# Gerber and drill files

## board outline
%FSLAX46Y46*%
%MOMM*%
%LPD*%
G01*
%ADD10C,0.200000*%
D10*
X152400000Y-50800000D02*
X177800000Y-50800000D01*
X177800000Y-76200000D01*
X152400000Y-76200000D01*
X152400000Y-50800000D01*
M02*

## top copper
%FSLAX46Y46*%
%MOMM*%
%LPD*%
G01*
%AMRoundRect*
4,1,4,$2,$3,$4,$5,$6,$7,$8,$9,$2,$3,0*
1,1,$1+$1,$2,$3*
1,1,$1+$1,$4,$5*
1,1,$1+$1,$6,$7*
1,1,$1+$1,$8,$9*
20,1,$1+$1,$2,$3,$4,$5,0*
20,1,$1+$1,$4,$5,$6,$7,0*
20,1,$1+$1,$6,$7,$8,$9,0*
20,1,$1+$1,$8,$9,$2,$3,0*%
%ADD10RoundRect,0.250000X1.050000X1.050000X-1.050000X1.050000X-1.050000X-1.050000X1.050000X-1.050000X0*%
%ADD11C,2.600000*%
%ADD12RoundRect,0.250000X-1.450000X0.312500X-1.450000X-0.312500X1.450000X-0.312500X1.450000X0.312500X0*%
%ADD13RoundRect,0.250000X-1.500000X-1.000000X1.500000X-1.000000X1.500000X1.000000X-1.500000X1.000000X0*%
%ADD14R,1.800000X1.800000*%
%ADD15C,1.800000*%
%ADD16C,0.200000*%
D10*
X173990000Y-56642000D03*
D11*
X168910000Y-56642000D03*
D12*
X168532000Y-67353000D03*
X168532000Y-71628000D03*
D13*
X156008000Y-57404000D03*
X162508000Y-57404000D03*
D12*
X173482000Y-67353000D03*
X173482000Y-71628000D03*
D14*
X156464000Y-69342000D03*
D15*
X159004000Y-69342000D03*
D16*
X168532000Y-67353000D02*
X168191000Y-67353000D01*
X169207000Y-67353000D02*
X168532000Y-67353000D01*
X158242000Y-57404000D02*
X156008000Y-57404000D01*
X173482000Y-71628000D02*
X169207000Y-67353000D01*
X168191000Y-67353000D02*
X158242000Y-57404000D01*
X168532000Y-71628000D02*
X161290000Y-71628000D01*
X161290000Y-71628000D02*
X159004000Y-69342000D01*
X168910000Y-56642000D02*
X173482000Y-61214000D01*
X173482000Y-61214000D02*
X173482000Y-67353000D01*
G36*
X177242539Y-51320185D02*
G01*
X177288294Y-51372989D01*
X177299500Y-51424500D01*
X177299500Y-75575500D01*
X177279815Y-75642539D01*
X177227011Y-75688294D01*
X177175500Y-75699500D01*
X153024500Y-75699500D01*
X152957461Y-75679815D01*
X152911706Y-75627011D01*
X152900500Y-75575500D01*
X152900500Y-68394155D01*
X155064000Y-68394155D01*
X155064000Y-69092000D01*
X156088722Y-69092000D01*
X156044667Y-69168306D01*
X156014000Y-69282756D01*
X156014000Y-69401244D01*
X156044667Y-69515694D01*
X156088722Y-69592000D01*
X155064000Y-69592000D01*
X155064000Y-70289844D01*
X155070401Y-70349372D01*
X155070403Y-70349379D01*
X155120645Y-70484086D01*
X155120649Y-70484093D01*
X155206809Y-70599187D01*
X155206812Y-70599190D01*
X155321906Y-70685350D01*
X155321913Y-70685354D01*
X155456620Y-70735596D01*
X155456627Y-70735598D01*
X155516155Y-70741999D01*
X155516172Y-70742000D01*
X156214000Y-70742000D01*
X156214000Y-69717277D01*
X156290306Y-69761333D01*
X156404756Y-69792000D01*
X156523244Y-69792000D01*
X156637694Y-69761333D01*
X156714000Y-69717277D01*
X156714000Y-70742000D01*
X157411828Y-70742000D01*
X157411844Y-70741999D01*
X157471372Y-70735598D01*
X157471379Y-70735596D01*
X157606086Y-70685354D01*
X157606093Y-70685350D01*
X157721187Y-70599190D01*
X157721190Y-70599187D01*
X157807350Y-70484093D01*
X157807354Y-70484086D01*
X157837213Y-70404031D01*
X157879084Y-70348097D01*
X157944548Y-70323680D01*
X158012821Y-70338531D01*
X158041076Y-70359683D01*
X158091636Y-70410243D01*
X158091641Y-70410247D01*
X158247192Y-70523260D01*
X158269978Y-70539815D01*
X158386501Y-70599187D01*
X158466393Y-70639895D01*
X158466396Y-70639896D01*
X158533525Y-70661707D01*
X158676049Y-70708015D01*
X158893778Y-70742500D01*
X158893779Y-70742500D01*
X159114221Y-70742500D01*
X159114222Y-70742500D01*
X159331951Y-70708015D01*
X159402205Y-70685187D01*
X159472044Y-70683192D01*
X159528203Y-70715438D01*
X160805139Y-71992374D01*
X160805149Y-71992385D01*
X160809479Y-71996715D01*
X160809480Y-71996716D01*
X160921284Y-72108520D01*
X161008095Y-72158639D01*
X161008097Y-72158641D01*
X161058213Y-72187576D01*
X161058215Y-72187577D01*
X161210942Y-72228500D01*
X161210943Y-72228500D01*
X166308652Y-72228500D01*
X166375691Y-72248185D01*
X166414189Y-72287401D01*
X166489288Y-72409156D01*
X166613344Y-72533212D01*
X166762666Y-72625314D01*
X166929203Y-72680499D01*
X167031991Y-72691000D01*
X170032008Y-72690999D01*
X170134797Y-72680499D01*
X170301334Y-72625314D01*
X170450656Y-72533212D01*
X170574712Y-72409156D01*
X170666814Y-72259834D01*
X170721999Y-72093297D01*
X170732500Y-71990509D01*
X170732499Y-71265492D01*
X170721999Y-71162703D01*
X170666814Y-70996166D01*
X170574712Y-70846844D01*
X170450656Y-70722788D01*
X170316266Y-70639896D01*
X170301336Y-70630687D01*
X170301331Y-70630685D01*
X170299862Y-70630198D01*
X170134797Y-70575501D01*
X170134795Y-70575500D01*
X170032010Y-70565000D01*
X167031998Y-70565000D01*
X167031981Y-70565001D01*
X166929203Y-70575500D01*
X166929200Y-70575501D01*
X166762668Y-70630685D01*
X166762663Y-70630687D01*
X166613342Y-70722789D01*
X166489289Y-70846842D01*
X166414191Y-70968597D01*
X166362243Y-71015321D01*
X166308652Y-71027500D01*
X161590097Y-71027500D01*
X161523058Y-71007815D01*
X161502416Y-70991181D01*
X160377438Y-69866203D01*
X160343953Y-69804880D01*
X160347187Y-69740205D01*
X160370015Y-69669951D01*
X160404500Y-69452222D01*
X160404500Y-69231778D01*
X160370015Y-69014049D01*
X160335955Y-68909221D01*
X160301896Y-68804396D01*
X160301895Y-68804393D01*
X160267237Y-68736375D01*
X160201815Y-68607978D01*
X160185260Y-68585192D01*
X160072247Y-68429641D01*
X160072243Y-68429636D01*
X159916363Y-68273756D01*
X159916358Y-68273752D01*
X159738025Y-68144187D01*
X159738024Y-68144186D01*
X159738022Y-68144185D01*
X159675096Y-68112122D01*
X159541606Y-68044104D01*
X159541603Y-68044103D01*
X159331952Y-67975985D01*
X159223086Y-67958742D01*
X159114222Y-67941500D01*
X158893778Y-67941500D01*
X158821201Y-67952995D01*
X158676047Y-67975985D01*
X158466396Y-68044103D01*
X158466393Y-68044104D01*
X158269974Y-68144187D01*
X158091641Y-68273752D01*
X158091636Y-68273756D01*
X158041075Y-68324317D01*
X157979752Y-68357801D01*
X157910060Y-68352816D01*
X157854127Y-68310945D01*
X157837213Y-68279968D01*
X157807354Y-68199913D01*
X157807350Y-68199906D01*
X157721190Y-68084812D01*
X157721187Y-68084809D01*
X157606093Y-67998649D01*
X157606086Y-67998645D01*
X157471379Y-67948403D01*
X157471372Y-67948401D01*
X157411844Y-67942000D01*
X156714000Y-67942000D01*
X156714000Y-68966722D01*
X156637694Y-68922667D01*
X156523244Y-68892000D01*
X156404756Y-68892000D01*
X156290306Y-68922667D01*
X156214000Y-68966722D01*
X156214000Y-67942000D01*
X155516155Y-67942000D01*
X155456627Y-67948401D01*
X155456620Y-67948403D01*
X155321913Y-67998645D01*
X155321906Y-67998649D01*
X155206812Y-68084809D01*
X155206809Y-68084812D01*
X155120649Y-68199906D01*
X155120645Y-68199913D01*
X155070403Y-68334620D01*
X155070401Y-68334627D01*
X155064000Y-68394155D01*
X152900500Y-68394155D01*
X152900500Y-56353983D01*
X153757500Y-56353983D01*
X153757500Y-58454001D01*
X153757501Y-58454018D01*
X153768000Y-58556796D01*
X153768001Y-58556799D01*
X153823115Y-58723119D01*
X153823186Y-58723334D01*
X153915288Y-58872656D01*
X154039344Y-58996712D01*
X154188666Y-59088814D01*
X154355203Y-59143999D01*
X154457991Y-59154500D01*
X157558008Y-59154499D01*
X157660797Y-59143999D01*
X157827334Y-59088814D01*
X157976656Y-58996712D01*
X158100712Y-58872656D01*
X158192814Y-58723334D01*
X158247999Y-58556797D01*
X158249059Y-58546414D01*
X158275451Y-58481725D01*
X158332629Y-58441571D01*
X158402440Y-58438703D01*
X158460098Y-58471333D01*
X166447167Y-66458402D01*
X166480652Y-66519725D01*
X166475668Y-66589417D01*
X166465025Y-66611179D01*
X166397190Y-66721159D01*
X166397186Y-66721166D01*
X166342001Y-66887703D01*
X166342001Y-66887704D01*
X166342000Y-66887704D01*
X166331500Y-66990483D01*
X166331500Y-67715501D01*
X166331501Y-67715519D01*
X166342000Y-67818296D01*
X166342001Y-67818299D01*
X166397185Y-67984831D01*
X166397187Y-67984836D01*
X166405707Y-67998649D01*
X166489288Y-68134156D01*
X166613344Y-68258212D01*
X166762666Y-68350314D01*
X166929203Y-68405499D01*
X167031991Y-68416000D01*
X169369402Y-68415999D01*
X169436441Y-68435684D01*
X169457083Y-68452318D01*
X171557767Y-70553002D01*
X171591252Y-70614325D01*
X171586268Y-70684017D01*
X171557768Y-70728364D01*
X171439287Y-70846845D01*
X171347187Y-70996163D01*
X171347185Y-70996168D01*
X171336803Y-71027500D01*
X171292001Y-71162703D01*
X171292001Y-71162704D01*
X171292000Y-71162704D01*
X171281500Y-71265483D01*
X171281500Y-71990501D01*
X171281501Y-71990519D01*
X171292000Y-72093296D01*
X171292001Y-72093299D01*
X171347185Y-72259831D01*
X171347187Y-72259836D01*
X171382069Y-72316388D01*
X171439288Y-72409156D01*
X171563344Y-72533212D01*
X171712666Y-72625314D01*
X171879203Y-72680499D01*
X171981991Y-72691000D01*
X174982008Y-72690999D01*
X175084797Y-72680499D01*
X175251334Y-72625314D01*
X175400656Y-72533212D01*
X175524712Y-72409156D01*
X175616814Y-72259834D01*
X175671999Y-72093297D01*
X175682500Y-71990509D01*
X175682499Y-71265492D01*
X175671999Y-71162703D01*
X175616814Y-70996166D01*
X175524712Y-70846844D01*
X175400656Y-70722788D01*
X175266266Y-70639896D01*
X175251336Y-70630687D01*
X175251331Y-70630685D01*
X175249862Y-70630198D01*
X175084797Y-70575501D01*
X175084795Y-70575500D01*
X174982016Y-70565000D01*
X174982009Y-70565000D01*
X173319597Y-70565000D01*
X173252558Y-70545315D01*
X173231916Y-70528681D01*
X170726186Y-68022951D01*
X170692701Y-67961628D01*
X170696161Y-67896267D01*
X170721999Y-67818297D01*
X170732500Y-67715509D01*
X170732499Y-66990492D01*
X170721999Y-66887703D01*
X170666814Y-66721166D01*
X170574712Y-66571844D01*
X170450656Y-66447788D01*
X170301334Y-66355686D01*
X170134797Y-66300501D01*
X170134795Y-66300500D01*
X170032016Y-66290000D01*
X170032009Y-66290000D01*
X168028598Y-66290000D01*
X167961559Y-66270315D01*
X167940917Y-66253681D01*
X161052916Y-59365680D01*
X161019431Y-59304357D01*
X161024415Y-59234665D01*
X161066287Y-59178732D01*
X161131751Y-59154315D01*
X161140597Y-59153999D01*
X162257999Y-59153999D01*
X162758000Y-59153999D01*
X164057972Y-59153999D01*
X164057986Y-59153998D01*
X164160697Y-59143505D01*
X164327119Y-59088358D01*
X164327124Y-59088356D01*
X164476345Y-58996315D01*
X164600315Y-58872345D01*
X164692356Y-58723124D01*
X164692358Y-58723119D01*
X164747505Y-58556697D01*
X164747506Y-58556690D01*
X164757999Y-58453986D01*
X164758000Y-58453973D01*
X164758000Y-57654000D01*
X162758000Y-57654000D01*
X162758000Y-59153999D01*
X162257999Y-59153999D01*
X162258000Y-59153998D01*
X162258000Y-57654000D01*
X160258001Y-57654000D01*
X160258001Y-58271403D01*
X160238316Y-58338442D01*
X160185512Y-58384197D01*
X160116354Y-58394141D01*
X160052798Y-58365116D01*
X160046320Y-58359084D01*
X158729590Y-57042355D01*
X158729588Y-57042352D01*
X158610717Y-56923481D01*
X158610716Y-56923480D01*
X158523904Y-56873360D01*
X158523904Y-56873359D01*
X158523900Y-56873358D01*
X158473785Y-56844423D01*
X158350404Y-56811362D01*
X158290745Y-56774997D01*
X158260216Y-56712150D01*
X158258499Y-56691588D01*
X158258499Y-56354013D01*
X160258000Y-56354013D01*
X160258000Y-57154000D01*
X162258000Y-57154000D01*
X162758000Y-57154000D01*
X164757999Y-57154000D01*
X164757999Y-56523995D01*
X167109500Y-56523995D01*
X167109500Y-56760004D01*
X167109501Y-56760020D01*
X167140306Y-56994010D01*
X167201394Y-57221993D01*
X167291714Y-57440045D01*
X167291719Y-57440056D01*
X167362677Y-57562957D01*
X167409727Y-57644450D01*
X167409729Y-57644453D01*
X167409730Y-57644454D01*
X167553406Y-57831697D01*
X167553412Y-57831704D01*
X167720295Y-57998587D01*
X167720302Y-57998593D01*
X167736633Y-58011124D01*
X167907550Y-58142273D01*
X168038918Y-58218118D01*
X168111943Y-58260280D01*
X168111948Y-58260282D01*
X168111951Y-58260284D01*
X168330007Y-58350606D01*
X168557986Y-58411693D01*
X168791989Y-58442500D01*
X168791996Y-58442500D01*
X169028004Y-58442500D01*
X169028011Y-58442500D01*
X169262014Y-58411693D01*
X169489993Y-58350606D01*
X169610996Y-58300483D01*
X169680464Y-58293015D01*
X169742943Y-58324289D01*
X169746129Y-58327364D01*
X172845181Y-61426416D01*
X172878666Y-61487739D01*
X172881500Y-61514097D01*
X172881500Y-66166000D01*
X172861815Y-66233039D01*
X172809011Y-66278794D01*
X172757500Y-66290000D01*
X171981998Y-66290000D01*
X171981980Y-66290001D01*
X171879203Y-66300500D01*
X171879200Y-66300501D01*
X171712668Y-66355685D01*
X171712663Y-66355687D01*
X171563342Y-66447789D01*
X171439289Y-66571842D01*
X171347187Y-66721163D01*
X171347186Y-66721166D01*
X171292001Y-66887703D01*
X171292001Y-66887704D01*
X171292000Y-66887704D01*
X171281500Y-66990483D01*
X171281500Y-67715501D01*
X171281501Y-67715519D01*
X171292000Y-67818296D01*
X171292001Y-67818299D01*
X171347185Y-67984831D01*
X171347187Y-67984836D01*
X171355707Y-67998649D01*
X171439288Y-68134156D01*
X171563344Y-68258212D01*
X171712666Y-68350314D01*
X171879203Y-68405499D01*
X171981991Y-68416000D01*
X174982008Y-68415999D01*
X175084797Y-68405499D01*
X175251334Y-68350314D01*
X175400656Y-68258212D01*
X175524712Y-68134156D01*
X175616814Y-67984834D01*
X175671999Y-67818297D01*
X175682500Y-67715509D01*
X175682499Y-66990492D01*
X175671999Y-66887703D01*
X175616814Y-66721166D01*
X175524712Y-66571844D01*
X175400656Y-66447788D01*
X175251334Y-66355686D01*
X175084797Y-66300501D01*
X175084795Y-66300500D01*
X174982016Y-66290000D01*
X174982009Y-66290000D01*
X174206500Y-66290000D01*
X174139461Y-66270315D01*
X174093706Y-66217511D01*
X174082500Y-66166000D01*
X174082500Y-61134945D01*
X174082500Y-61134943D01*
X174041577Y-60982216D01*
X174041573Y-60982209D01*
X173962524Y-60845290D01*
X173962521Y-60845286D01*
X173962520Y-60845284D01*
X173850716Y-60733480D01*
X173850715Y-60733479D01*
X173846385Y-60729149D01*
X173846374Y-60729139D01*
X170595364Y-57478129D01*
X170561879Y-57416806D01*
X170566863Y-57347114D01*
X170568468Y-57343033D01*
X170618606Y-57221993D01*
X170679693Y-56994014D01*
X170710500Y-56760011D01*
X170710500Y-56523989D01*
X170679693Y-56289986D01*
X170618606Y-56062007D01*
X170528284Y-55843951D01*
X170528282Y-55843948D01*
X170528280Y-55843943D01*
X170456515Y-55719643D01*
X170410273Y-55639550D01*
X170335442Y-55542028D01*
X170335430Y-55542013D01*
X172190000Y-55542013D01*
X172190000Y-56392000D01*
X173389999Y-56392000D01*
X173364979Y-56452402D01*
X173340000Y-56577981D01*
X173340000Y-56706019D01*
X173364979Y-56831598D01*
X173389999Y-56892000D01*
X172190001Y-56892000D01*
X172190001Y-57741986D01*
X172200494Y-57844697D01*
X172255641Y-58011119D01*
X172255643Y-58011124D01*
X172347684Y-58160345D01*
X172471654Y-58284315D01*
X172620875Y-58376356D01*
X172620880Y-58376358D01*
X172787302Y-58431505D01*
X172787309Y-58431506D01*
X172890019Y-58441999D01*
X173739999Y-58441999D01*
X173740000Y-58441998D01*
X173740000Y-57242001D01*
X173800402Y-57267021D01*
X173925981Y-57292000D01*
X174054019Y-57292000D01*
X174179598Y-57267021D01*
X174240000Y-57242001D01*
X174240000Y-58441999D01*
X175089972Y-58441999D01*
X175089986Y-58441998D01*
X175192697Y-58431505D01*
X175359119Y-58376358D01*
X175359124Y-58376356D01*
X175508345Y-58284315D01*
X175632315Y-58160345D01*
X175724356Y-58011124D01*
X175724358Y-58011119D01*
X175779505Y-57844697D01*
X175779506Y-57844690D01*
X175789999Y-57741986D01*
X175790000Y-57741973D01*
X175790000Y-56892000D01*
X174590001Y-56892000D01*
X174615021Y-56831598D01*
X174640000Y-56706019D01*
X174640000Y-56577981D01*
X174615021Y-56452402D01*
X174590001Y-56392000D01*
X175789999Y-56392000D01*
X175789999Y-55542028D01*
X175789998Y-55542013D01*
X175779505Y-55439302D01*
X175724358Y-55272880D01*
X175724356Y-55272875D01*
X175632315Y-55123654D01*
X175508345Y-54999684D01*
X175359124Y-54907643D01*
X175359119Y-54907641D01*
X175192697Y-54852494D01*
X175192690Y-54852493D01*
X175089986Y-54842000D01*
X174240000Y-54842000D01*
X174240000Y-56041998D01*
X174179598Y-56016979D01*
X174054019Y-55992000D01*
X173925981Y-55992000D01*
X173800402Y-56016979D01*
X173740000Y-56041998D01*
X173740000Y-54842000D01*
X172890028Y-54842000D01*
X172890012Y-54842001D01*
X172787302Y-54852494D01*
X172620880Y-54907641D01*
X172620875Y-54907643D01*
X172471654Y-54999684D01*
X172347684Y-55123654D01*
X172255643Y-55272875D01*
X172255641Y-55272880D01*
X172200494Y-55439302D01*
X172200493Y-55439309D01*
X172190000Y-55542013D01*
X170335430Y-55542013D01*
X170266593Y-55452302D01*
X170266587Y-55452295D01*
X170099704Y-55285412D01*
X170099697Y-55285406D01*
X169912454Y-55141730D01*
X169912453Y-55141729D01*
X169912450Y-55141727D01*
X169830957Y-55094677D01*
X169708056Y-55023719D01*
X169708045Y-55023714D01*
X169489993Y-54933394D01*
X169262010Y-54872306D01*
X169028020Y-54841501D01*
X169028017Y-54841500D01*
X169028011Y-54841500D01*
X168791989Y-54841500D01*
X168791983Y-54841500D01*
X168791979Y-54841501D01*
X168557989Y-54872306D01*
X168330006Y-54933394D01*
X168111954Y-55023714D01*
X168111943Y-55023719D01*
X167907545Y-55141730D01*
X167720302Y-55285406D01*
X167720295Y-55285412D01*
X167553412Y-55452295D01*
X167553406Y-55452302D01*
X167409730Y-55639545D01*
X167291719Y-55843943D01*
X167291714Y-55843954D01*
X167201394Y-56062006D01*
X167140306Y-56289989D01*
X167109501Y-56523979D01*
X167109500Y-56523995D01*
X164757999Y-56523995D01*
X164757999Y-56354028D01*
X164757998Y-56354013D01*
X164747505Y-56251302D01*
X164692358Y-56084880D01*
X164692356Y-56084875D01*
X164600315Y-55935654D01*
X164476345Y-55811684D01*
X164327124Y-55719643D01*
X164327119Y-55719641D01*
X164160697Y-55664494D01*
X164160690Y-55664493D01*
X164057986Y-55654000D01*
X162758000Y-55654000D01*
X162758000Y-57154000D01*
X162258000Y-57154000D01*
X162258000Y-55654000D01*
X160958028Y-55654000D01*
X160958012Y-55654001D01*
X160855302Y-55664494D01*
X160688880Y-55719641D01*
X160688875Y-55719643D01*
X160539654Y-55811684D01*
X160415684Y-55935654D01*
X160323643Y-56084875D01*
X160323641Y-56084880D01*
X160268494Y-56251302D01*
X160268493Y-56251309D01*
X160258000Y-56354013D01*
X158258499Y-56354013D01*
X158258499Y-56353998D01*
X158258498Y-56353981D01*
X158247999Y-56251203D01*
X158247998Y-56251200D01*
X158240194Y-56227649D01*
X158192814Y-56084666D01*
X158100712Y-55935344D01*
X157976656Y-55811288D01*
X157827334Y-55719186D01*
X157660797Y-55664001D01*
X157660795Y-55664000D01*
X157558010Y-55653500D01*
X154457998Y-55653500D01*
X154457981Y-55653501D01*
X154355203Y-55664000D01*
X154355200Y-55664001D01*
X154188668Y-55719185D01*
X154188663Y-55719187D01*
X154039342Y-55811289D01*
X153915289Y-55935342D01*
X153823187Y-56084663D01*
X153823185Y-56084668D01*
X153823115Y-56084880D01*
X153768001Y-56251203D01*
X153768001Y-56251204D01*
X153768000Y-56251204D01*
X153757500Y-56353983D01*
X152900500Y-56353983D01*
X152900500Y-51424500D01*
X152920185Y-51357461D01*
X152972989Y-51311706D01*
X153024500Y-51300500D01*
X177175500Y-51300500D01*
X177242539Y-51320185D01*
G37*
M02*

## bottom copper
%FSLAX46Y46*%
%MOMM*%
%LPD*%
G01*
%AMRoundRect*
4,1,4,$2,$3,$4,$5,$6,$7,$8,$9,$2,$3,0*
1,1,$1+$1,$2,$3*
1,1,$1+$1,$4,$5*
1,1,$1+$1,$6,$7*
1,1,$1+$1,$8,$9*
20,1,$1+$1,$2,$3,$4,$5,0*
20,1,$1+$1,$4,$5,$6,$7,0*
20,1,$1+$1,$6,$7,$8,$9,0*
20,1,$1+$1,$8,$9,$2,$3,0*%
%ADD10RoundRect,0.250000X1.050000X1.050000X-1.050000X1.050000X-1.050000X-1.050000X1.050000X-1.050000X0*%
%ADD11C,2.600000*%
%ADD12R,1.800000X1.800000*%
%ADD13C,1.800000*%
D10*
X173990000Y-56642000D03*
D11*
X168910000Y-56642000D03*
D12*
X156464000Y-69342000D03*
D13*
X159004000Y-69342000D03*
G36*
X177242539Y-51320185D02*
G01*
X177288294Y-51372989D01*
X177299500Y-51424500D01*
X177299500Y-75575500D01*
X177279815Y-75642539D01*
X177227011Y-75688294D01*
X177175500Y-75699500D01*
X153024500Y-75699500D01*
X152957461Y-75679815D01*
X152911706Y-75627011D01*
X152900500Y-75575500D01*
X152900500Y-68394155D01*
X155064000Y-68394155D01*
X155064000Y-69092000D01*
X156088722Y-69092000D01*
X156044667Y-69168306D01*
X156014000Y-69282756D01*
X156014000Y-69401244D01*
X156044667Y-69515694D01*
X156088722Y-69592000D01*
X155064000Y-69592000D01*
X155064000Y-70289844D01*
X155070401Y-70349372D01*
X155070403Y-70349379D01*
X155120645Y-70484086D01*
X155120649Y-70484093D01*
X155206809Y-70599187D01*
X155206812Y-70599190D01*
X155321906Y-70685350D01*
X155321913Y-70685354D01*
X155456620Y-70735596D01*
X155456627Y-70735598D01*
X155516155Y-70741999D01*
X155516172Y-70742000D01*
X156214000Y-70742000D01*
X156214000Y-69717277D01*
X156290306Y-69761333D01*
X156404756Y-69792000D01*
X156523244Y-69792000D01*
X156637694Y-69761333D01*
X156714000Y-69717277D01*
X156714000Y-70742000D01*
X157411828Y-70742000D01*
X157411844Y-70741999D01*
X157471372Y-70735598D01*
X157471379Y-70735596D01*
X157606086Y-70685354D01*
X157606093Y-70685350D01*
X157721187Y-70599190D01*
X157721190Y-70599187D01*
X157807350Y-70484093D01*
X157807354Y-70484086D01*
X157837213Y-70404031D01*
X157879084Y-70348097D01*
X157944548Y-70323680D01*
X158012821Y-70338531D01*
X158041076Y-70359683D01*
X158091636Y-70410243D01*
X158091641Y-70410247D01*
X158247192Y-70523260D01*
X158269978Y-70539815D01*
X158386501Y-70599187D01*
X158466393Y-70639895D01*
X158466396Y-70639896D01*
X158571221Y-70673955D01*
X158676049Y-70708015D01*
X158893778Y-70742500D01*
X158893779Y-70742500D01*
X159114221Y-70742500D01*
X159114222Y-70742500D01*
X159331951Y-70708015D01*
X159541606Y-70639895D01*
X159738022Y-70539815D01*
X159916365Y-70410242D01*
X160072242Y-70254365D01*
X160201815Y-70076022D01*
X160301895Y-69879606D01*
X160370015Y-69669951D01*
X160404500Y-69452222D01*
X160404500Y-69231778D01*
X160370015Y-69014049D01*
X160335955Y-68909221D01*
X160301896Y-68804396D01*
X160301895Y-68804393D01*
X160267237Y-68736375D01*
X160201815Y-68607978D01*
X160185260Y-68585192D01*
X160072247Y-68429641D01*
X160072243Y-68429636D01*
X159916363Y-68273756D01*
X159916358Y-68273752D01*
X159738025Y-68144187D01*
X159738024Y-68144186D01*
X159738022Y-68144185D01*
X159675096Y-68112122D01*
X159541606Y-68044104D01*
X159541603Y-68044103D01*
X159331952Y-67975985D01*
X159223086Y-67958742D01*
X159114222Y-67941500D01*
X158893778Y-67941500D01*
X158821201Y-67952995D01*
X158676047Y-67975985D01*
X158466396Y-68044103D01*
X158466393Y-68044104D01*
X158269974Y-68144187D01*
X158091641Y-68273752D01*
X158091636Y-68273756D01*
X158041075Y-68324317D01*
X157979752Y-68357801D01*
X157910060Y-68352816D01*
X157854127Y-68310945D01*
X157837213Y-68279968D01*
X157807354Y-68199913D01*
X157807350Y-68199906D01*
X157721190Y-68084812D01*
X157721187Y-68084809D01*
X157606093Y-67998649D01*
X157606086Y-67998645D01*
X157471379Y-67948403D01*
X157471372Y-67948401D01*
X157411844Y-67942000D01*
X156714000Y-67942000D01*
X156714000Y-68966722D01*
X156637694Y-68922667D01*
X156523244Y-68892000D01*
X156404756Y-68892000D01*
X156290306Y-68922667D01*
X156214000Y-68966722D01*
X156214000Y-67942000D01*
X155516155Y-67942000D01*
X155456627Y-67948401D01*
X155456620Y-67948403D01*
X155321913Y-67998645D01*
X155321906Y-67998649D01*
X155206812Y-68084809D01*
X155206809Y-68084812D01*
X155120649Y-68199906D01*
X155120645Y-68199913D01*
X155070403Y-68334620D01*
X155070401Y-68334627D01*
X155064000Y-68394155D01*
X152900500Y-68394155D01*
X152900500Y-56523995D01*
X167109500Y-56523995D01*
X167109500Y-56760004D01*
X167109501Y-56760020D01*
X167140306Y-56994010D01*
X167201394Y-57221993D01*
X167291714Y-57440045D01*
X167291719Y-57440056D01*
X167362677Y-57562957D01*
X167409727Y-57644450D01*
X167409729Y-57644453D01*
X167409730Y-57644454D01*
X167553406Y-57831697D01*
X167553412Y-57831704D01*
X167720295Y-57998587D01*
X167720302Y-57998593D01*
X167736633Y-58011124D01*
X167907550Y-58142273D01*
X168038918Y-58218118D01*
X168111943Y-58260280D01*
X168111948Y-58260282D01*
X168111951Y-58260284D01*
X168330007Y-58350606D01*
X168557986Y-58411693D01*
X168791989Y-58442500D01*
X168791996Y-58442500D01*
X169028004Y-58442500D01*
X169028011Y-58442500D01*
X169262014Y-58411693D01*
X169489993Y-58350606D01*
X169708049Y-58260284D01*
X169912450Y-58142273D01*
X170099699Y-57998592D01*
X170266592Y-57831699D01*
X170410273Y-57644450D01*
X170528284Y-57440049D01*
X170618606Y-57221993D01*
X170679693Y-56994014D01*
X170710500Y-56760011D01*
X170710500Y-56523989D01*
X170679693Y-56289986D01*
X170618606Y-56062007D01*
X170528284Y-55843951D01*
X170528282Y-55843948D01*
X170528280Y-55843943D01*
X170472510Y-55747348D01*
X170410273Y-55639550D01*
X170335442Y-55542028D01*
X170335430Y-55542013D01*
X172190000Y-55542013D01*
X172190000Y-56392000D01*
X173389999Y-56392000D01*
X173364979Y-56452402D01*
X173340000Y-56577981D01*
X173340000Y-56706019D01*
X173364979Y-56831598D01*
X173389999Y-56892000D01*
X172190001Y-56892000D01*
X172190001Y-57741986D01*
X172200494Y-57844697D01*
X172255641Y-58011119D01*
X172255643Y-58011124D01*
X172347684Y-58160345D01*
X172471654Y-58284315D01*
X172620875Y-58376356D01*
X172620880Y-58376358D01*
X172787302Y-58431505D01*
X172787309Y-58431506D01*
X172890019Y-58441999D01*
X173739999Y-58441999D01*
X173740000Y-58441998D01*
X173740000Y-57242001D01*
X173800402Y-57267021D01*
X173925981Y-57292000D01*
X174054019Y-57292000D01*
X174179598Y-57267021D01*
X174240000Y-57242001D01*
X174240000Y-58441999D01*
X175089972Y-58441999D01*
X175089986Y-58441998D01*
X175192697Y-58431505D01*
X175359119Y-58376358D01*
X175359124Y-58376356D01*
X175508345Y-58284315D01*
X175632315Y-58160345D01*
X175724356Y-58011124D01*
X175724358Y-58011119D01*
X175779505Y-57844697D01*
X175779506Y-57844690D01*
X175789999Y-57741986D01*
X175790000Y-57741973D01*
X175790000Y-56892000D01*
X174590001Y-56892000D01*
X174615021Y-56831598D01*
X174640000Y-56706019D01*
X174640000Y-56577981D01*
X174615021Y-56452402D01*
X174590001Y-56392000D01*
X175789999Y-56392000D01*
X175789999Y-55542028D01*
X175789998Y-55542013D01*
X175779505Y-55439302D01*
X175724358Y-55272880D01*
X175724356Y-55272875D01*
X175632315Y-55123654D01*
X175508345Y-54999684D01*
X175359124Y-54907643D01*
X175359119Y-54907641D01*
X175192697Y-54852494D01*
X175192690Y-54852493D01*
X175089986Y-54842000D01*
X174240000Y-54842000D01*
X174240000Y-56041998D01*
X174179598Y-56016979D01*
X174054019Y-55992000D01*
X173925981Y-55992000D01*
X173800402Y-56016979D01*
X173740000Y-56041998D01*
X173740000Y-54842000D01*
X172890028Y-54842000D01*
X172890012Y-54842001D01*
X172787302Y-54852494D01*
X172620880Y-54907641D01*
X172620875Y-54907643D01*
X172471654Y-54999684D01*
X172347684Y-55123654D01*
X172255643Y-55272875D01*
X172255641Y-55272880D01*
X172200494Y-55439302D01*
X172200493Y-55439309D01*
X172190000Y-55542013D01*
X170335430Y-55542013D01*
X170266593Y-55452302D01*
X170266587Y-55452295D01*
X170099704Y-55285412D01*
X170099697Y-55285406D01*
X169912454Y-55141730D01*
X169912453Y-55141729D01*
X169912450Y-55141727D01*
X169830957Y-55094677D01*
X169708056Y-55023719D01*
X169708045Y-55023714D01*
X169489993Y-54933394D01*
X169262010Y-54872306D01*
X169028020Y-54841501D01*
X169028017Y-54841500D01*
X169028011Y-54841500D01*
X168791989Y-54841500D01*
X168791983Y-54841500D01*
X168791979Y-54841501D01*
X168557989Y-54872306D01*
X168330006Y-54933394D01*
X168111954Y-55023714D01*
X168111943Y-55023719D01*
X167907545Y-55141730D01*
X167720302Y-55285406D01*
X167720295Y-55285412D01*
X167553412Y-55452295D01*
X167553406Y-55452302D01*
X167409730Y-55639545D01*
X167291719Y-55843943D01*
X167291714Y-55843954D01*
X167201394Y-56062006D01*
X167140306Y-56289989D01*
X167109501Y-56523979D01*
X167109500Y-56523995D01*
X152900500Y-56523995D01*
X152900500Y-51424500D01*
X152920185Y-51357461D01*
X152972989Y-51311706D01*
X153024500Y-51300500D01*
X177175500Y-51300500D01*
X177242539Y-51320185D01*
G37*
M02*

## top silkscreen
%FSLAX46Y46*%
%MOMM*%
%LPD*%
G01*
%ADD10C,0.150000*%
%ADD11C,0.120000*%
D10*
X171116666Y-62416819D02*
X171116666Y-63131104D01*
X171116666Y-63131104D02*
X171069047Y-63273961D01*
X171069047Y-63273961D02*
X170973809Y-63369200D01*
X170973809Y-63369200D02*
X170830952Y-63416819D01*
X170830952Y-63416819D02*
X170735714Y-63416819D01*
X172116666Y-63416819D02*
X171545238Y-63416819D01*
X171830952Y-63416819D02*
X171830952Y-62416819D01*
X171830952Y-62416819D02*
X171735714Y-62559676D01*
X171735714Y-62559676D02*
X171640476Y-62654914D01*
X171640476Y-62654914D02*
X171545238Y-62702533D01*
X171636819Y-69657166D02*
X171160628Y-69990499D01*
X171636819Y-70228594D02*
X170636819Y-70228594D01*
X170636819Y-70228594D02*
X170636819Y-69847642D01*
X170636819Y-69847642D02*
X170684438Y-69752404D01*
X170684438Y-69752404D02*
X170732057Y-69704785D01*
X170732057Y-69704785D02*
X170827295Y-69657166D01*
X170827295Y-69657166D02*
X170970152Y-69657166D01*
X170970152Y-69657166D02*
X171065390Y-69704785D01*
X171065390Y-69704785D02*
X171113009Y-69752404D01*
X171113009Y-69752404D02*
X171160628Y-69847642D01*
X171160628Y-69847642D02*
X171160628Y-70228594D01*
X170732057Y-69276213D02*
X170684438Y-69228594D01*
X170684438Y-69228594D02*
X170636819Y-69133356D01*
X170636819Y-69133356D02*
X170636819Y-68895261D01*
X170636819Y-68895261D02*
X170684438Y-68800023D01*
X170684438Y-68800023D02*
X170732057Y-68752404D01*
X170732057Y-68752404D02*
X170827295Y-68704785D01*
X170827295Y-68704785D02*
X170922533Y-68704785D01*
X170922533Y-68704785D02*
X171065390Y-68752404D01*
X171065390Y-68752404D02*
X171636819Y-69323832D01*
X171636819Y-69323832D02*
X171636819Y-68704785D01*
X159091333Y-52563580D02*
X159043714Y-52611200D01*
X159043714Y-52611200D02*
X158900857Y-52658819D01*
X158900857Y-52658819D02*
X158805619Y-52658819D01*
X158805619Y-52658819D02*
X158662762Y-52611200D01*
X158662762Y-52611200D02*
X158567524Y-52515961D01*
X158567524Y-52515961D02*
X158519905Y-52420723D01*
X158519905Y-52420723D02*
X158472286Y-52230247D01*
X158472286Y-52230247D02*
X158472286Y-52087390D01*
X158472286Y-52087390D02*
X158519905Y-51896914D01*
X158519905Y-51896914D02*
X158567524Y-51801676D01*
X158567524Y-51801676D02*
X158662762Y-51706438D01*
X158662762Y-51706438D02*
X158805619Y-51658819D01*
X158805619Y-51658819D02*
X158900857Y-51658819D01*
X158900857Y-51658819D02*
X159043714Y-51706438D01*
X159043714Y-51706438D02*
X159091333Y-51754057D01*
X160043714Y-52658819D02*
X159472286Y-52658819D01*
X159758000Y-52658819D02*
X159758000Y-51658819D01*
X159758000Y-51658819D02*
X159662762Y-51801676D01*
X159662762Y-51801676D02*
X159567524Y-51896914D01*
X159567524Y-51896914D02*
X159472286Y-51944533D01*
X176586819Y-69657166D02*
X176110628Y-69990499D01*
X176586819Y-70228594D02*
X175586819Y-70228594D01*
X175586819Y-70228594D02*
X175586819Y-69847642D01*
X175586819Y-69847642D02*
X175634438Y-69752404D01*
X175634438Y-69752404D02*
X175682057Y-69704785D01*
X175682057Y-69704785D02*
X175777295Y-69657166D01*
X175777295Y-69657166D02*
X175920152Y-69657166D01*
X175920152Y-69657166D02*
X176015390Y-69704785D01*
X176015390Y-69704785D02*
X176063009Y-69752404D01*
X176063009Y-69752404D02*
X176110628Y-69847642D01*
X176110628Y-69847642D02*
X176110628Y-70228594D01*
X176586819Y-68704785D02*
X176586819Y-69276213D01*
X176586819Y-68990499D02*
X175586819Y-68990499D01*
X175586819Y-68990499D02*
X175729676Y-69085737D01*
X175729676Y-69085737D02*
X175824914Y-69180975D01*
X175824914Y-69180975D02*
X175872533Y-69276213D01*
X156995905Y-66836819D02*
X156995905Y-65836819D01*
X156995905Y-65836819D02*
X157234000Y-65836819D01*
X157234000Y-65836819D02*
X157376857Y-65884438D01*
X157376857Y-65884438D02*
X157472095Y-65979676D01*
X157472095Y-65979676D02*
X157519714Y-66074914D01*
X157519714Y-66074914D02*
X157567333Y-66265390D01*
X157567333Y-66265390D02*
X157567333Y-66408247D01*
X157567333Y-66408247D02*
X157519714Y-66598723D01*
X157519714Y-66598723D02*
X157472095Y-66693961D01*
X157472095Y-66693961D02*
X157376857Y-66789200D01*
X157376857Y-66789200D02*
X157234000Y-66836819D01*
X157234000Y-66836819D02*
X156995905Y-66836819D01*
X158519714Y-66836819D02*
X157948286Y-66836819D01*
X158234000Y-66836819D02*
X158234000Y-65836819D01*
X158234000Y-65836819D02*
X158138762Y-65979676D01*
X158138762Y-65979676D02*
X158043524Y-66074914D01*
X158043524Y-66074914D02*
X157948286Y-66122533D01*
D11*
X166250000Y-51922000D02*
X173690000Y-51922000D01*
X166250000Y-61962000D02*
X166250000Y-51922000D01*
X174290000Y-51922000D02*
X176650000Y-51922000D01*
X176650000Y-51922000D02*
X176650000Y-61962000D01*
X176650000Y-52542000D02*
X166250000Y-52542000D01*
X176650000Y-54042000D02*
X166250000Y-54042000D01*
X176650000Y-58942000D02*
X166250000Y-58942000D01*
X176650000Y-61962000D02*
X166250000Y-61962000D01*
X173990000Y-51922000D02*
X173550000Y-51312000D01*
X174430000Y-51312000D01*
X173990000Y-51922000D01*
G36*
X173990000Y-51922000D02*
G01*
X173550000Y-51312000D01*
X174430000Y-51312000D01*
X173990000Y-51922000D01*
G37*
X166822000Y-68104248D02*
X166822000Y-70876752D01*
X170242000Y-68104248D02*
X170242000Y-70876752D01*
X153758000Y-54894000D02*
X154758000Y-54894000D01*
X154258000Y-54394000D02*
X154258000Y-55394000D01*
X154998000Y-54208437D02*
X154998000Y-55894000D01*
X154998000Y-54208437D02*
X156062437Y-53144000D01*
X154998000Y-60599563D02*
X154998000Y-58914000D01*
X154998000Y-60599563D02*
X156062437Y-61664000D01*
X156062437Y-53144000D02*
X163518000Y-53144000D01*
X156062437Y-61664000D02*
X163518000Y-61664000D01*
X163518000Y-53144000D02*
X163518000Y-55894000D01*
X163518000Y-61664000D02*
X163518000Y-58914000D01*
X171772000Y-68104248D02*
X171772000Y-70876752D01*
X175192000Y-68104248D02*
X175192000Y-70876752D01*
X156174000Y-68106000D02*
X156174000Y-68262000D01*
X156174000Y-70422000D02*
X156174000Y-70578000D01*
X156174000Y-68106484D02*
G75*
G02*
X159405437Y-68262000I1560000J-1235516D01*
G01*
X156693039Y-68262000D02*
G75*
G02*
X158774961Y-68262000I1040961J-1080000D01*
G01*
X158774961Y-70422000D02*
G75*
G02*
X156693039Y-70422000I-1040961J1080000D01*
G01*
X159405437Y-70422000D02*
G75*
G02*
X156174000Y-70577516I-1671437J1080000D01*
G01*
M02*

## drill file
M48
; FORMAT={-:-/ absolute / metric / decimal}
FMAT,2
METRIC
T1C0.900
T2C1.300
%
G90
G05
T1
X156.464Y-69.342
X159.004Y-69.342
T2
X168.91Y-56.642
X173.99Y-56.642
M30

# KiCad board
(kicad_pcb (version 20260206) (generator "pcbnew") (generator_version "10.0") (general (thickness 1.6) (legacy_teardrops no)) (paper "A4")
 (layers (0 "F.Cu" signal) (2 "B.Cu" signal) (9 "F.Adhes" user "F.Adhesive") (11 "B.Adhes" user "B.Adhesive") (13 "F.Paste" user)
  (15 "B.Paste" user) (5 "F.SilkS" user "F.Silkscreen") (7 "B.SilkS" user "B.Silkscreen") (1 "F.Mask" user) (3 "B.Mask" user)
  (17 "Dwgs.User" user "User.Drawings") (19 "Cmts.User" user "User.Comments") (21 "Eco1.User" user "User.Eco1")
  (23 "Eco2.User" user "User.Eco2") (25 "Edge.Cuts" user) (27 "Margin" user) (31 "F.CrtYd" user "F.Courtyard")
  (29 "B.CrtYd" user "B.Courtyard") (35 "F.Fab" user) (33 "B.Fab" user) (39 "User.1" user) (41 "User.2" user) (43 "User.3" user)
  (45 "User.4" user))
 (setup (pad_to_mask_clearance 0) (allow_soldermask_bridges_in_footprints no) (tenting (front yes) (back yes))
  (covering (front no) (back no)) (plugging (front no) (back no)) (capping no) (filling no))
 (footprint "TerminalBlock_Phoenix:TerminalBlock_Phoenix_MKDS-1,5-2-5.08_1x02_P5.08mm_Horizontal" (layer "F.Cu") (at 173.99 56.642 180)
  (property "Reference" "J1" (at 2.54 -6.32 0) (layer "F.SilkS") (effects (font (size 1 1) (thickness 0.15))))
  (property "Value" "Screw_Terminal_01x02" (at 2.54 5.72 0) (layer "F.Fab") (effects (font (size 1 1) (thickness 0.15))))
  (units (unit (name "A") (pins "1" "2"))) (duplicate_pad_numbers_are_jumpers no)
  (fp_line (start 7.74 4.72) (end 0.3 4.72) (stroke (width 0.12) (type solid)) (layer "F.SilkS"))
  (fp_line (start 7.74 -5.32) (end 7.74 4.72) (stroke (width 0.12) (type solid)) (layer "F.SilkS"))
  (fp_line (start -0.3 4.72) (end -2.66 4.72) (stroke (width 0.12) (type solid)) (layer "F.SilkS"))
  (fp_line (start -2.66 4.72) (end -2.66 -5.32) (stroke (width 0.12) (type solid)) (layer "F.SilkS"))
  (fp_line (start -2.66 4.1) (end 7.74 4.1) (stroke (width 0.12) (type solid)) (layer "F.SilkS"))
  (fp_line (start -2.66 2.6) (end 7.74 2.6) (stroke (width 0.12) (type solid)) (layer "F.SilkS"))
  (fp_line (start -2.66 -2.3) (end 7.74 -2.3) (stroke (width 0.12) (type solid)) (layer "F.SilkS"))
  (fp_line (start -2.66 -5.32) (end 7.74 -5.32) (stroke (width 0.12) (type solid)) (layer "F.SilkS"))
  (fp_poly (pts (xy 0 4.72) (xy 0.44 5.33) (xy -0.44 5.33)) (stroke (width 0.12) (type solid)) (fill yes) (layer "F.SilkS"))
  (pad "1" thru_hole roundrect (at 0 0 180) (size 2.6 2.6) (drill 1.3) (layers "*.Cu" "*.Mask") (remove_unused_layers no)
   (roundrect_rratio 0.096154) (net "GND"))
  (pad "2" thru_hole circle (at 5.08 0 180) (size 2.6 2.6) (drill 1.3) (layers "*.Cu" "*.Mask") (remove_unused_layers no)
   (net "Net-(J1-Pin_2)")))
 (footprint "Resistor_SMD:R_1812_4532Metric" (layer "F.Cu") (at 168.532 69.4905 -90)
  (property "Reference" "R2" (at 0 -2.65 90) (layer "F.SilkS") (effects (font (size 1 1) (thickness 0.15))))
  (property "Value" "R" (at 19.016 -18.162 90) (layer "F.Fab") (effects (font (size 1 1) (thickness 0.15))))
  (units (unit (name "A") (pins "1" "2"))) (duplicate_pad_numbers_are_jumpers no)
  (fp_line (start -1.386252 1.71) (end 1.386252 1.71) (stroke (width 0.12) (type solid)) (layer "F.SilkS"))
  (fp_line (start -1.386252 -1.71) (end 1.386252 -1.71) (stroke (width 0.12) (type solid)) (layer "F.SilkS"))
  (pad "1" smd roundrect (at -2.1375 0 270) (size 1.125 3.4) (layers "F.Cu" "F.Mask" "F.Paste") (roundrect_rratio 0.222222)
   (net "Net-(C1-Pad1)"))
  (pad "2" smd roundrect (at 2.1375 0 270) (size 1.125 3.4) (layers "F.Cu" "F.Mask" "F.Paste") (roundrect_rratio 0.222222)
   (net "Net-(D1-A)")))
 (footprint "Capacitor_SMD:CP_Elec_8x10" (layer "F.Cu") (at 159.258 57.404)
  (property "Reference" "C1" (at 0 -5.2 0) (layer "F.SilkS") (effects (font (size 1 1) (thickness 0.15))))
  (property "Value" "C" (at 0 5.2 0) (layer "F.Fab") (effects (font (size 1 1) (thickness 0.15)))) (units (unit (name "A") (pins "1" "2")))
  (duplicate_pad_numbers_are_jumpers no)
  (fp_line (start -5.5 -2.51) (end -4.5 -2.51) (stroke (width 0.12) (type solid)) (layer "F.SilkS"))
  (fp_line (start -5 -3.01) (end -5 -2.01) (stroke (width 0.12) (type solid)) (layer "F.SilkS"))
  (fp_line (start -4.26 -3.195563) (end -4.26 -1.51) (stroke (width 0.12) (type solid)) (layer "F.SilkS"))
  (fp_line (start -4.26 -3.195563) (end -3.195563 -4.26) (stroke (width 0.12) (type solid)) (layer "F.SilkS"))
  (fp_line (start -4.26 3.195563) (end -4.26 1.51) (stroke (width 0.12) (type solid)) (layer "F.SilkS"))
  (fp_line (start -4.26 3.195563) (end -3.195563 4.26) (stroke (width 0.12) (type solid)) (layer "F.SilkS"))
  (fp_line (start -3.195563 -4.26) (end 4.26 -4.26) (stroke (width 0.12) (type solid)) (layer "F.SilkS"))
  (fp_line (start -3.195563 4.26) (end 4.26 4.26) (stroke (width 0.12) (type solid)) (layer "F.SilkS"))
  (fp_line (start 4.26 -4.26) (end 4.26 -1.51) (stroke (width 0.12) (type solid)) (layer "F.SilkS"))
  (fp_line (start 4.26 4.26) (end 4.26 1.51) (stroke (width 0.12) (type solid)) (layer "F.SilkS"))
  (pad "1" smd roundrect (at -3.25 0) (size 3.5 2.5) (layers "F.Cu" "F.Mask" "F.Paste") (roundrect_rratio 0.1) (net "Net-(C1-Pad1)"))
  (pad "2" smd roundrect (at 3.25 0) (size 3.5 2.5) (layers "F.Cu" "F.Mask" "F.Paste") (roundrect_rratio 0.1) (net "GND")))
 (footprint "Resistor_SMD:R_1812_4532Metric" (layer "F.Cu") (at 173.482 69.4905 -90)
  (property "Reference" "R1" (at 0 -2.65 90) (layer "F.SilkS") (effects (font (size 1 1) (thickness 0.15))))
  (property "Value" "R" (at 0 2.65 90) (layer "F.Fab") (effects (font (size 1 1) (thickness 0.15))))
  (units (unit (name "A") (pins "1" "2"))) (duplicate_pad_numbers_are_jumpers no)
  (fp_line (start -1.386252 1.71) (end 1.386252 1.71) (stroke (width 0.12) (type solid)) (layer "F.SilkS"))
  (fp_line (start -1.386252 -1.71) (end 1.386252 -1.71) (stroke (width 0.12) (type solid)) (layer "F.SilkS"))
  (pad "1" smd roundrect (at -2.1375 0 270) (size 1.125 3.4) (layers "F.Cu" "F.Mask" "F.Paste") (roundrect_rratio 0.222222)
   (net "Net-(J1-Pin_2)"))
  (pad "2" smd roundrect (at 2.1375 0 270) (size 1.125 3.4) (layers "F.Cu" "F.Mask" "F.Paste") (roundrect_rratio 0.222222)
   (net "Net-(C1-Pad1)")))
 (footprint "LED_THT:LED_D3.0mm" (layer "F.Cu") (at 156.464 69.342)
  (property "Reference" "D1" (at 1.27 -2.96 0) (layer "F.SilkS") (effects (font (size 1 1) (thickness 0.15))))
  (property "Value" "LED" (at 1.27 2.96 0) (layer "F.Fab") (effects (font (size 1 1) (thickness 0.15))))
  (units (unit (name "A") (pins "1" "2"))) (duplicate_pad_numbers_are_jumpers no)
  (fp_line (start -0.29 -1.236) (end -0.29 -1.08) (stroke (width 0.12) (type solid)) (layer "F.SilkS"))
  (fp_line (start -0.29 1.08) (end -0.29 1.236) (stroke (width 0.12) (type solid)) (layer "F.SilkS"))
  (fp_arc (start -0.29 -1.235516) (mid 1.36566 -1.987699) (end 2.941437 -1.08) (stroke (width 0.12) (type solid)) (layer "F.SilkS"))
  (fp_arc (start 0.229039 -1.08) (mid 1.27 -1.5) (end 2.310961 -1.08) (stroke (width 0.12) (type solid)) (layer "F.SilkS"))
  (fp_arc (start 2.310961 1.08) (mid 1.27 1.5) (end 0.229039 1.08) (stroke (width 0.12) (type solid)) (layer "F.SilkS"))
  (fp_arc (start 2.941437 1.08) (mid 1.36566 1.987699) (end -0.29 1.235516) (stroke (width 0.12) (type solid)) (layer "F.SilkS"))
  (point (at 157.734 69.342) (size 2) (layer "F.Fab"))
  (pad "1" thru_hole rect (at 0 0) (size 1.8 1.8) (drill 0.9) (layers "*.Cu" "*.Mask") (remove_unused_layers no) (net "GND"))
  (pad "2" thru_hole circle (at 2.54 0) (size 1.8 1.8) (drill 0.9) (layers "*.Cu" "*.Mask") (remove_unused_layers no) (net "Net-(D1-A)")))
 (gr_poly
  (pts (xy 152.4 50.8) (xy 177.8 50.8) (xy 177.8 76.2) (xy 152.4 76.2)) (stroke (width 0.2) (type solid)) (fill no) (layer "Edge.Cuts"))
 (segment (start 168.532 67.353) (end 168.191 67.353) (width 0.2) (layer "F.Cu") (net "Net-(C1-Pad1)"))
 (segment (start 169.207 67.353) (end 168.532 67.353) (width 0.2) (layer "F.Cu") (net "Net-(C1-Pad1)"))
 (segment (start 158.242 57.404) (end 156.008 57.404) (width 0.2) (layer "F.Cu") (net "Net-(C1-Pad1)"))
 (segment (start 173.482 71.628) (end 169.207 67.353) (width 0.2) (layer "F.Cu") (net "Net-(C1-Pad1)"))
 (segment (start 168.191 67.353) (end 158.242 57.404) (width 0.2) (layer "F.Cu") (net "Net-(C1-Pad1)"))
 (segment (start 168.532 71.628) (end 161.29 71.628) (width 0.2) (layer "F.Cu") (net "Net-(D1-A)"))
 (segment (start 161.29 71.628) (end 159.004 69.342) (width 0.2) (layer "F.Cu") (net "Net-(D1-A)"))
 (segment (start 168.91 56.642) (end 173.482 61.214) (width 0.2) (layer "F.Cu") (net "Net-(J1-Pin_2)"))
 (segment (start 173.482 61.214) (end 173.482 67.353) (width 0.2) (layer "F.Cu") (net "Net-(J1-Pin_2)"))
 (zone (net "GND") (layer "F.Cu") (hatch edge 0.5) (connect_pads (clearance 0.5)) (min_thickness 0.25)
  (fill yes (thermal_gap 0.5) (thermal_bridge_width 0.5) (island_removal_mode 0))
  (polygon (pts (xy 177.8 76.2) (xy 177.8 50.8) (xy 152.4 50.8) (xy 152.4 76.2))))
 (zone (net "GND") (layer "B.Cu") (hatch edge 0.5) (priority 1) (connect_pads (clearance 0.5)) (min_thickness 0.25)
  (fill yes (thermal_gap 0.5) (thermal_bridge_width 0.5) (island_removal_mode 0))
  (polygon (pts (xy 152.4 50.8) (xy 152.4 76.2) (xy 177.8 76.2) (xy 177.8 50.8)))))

